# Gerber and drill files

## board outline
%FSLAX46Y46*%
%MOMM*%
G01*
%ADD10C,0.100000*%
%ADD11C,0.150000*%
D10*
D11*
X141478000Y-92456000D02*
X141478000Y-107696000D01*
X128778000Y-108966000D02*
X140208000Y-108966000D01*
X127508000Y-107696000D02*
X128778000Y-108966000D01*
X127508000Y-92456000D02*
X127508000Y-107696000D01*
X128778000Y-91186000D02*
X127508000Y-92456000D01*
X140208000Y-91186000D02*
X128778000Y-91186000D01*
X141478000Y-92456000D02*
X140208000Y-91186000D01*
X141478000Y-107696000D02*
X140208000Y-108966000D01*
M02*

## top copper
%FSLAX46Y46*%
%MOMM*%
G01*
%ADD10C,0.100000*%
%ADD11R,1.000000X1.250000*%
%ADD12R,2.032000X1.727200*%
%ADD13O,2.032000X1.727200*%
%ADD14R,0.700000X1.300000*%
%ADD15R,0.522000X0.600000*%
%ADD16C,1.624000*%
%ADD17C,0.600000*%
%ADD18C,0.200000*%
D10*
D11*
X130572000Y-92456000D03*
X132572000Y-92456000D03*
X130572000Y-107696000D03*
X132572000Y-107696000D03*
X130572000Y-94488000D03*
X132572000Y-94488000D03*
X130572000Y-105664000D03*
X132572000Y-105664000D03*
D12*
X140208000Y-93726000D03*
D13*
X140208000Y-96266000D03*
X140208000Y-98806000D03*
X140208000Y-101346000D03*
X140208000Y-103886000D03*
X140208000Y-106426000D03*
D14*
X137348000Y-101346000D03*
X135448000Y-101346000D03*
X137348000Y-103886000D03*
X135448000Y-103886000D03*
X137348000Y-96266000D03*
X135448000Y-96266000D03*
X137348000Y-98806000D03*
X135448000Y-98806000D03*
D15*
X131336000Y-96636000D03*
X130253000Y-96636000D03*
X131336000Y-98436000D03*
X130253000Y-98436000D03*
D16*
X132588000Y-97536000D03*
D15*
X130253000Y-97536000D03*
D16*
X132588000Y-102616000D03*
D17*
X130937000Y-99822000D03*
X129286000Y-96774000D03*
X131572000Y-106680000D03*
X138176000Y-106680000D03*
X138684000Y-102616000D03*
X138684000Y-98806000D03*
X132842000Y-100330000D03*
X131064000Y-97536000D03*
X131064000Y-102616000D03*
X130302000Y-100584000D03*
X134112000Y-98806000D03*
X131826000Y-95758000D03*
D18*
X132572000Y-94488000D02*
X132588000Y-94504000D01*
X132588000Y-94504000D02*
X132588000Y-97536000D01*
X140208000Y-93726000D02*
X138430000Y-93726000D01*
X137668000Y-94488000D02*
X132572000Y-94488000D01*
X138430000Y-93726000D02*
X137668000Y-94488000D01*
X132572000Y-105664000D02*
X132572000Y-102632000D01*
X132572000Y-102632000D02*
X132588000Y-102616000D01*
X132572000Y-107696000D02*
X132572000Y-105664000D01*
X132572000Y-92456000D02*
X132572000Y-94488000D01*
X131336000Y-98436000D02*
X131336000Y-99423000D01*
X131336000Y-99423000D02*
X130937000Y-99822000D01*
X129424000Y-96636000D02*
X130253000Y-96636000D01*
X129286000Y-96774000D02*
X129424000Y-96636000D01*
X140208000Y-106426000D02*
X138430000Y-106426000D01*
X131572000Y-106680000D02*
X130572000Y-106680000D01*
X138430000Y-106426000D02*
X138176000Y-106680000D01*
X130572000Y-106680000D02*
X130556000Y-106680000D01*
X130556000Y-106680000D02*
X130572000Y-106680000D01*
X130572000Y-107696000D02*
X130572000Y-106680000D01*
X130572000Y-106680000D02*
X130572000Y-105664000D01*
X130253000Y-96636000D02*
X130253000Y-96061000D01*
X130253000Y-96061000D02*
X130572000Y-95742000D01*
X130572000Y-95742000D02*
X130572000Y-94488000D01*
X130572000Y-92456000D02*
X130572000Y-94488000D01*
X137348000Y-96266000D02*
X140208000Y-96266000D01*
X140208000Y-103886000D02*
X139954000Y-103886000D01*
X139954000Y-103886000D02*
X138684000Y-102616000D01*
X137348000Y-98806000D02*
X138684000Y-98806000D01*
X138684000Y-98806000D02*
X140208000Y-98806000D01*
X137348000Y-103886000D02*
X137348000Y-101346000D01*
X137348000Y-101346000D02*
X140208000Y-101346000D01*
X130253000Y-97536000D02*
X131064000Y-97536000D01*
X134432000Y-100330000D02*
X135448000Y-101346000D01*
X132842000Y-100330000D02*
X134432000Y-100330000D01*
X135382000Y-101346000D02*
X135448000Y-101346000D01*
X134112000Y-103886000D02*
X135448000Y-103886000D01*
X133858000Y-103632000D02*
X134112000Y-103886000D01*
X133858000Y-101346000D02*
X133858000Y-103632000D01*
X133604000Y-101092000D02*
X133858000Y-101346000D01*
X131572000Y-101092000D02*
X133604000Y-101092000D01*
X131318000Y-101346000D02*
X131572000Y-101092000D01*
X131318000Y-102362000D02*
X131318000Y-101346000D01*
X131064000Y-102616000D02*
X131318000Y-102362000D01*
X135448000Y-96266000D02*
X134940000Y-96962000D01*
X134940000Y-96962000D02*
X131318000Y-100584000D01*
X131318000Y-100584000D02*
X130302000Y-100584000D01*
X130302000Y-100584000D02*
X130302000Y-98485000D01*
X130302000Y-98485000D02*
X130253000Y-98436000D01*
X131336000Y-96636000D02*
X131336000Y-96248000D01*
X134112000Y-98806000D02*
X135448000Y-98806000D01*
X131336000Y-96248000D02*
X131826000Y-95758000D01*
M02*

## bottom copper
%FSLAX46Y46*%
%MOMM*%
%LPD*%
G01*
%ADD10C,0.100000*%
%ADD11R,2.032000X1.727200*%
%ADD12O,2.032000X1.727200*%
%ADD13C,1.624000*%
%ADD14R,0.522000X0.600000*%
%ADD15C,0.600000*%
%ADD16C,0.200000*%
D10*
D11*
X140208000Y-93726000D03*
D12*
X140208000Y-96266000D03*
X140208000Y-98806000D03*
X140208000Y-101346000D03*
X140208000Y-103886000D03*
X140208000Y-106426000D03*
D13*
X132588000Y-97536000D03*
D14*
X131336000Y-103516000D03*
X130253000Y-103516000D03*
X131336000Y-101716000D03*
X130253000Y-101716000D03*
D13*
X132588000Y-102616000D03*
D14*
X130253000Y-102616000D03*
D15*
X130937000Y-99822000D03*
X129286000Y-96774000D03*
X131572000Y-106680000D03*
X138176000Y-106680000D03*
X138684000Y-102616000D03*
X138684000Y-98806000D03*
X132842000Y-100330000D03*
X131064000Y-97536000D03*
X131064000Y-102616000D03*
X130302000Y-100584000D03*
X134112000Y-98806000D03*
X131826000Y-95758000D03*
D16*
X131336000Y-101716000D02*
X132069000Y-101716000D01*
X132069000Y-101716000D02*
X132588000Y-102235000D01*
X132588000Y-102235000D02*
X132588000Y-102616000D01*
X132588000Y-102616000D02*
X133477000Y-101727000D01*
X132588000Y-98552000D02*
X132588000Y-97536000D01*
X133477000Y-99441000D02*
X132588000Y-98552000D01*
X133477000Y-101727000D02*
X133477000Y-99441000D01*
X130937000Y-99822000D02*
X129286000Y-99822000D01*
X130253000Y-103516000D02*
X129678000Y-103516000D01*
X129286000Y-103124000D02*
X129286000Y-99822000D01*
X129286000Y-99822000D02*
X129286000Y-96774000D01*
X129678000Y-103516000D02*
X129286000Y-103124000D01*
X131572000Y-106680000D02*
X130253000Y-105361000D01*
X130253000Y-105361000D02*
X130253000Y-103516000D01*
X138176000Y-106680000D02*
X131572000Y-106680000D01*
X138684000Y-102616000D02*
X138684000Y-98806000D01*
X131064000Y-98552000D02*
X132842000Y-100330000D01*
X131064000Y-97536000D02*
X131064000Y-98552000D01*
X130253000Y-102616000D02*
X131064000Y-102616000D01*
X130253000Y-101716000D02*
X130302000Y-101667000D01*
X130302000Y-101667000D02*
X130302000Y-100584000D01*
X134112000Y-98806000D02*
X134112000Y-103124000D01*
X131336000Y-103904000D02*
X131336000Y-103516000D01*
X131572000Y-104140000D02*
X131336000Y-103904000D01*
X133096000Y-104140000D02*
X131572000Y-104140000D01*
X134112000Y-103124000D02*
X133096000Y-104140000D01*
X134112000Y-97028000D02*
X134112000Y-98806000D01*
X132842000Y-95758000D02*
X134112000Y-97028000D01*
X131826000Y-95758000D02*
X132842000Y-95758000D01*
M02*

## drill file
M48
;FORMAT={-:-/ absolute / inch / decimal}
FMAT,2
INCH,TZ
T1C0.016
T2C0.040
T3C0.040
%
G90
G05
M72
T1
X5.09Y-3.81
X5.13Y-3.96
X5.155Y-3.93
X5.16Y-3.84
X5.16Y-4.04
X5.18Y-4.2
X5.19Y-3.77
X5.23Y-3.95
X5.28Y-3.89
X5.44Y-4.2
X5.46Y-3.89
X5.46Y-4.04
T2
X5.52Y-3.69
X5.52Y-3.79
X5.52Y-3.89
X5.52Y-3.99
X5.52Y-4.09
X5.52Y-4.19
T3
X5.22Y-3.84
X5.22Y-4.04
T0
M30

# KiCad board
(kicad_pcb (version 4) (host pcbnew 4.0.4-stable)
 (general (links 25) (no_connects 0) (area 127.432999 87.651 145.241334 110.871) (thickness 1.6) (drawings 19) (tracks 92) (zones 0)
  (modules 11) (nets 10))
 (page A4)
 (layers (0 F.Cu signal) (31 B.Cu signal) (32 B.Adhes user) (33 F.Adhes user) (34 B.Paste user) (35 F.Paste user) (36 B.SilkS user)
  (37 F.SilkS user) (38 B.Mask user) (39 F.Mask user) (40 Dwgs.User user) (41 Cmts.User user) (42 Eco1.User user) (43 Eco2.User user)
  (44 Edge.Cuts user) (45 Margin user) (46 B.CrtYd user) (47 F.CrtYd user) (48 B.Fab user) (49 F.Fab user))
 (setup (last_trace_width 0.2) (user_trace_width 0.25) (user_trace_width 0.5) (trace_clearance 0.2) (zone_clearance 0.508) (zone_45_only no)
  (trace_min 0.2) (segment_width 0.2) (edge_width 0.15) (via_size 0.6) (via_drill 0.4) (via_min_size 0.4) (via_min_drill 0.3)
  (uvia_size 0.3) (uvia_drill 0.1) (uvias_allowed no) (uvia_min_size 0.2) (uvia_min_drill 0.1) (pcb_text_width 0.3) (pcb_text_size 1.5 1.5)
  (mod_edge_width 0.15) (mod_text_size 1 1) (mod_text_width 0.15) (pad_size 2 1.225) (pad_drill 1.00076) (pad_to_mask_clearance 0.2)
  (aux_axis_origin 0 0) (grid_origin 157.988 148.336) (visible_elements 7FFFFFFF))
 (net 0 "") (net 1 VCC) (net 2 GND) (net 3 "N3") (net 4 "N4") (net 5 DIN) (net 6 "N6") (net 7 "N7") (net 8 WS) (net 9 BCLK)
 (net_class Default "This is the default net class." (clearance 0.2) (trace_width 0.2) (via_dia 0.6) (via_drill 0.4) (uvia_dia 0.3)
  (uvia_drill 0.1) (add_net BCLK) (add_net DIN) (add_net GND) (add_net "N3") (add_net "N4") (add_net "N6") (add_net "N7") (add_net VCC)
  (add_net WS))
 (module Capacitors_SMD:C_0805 (layer F.Cu) (at 131.572 92.456)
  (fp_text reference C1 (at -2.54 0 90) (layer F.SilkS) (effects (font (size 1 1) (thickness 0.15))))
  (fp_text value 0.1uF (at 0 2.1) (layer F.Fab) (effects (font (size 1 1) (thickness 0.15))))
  (pad 1 smd rect (at -1 0) (size 1 1.25) (layers F.Cu F.Paste F.Mask) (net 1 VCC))
  (pad 2 smd rect (at 1 0) (size 1 1.25) (layers F.Cu F.Paste F.Mask) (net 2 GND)))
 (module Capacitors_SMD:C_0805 (layer F.Cu) (at 131.572 107.696)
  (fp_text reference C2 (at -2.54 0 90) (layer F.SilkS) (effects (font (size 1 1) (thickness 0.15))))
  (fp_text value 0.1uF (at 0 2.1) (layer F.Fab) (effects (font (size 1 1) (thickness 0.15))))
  (pad 1 smd rect (at -1 0) (size 1 1.25) (layers F.Cu F.Paste F.Mask) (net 1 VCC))
  (pad 2 smd rect (at 1 0) (size 1 1.25) (layers F.Cu F.Paste F.Mask) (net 2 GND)))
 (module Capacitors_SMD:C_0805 (layer F.Cu) (at 131.572 94.488)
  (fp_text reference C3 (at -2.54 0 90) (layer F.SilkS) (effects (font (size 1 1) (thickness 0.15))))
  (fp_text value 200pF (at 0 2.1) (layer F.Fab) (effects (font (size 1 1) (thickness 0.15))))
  (pad 1 smd rect (at -1 0) (size 1 1.25) (layers F.Cu F.Paste F.Mask) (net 1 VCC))
  (pad 2 smd rect (at 1 0) (size 1 1.25) (layers F.Cu F.Paste F.Mask) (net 2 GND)))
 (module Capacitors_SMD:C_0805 (layer F.Cu) (at 131.572 105.664)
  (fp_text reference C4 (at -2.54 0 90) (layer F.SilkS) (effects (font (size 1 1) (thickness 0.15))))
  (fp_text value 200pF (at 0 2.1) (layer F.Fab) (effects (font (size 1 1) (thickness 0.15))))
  (pad 1 smd rect (at -1 0) (size 1 1.25) (layers F.Cu F.Paste F.Mask) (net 1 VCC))
  (pad 2 smd rect (at 1 0) (size 1 1.25) (layers F.Cu F.Paste F.Mask) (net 2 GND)))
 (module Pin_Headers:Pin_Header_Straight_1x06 (layer F.Cu) (at 140.208 93.726)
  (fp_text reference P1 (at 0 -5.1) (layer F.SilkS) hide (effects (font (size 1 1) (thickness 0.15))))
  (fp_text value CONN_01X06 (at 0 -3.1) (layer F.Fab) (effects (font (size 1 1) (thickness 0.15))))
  (pad 1 thru_hole rect (at 0 0) (size 2.032 1.7272) (drill 1.016) (layers *.Cu *.Mask F.SilkS) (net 2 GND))
  (pad 2 thru_hole oval (at 0 2.54) (size 2.032 1.7272) (drill 1.016) (layers *.Cu *.Mask F.SilkS) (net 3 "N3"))
  (pad 3 thru_hole oval (at 0 5.08) (size 2.032 1.7272) (drill 1.016) (layers *.Cu *.Mask F.SilkS) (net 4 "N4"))
  (pad 4 thru_hole oval (at 0 7.62) (size 2.032 1.7272) (drill 1.016) (layers *.Cu *.Mask F.SilkS) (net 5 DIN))
  (pad 5 thru_hole oval (at 0 10.16) (size 2.032 1.7272) (drill 1.016) (layers *.Cu *.Mask F.SilkS) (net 4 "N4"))
  (pad 6 thru_hole oval (at 0 12.7) (size 2.032 1.7272) (drill 1.016) (layers *.Cu *.Mask F.SilkS) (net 1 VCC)))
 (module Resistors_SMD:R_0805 (layer F.Cu) (at 136.398 101.346 180)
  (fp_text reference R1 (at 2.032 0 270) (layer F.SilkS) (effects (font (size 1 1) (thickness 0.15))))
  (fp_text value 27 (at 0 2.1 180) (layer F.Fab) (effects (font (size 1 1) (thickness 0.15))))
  (pad 1 smd rect (at -0.95 0 180) (size 0.7 1.3) (layers F.Cu F.Paste F.Mask) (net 5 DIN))
  (pad 2 smd rect (at 0.95 0 180) (size 0.7 1.3) (layers F.Cu F.Paste F.Mask) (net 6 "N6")))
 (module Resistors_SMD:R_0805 (layer F.Cu) (at 136.398 103.886 180)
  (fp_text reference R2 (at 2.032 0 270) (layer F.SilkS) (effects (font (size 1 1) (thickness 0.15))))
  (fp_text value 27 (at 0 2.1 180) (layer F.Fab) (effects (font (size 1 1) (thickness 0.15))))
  (pad 1 smd rect (at -0.95 0 180) (size 0.7 1.3) (layers F.Cu F.Paste F.Mask) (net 5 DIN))
  (pad 2 smd rect (at 0.95 0 180) (size 0.7 1.3) (layers F.Cu F.Paste F.Mask) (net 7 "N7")))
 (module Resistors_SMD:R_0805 (layer F.Cu) (at 136.398 96.266 180)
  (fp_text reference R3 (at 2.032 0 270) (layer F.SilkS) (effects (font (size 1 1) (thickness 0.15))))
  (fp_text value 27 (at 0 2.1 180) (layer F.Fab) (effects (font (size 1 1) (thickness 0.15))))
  (pad 1 smd rect (at -0.95 0 180) (size 0.7 1.3) (layers F.Cu F.Paste F.Mask) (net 3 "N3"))
  (pad 2 smd rect (at 0.95 0 180) (size 0.7 1.3) (layers F.Cu F.Paste F.Mask) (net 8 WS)))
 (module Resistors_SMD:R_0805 (layer F.Cu) (at 136.398 98.806 180)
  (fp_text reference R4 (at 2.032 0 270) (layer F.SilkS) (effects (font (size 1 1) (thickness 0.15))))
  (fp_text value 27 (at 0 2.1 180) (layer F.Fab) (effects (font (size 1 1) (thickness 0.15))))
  (pad 1 smd rect (at -0.95 0 180) (size 0.7 1.3) (layers F.Cu F.Paste F.Mask) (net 4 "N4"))
  (pad 2 smd rect (at 0.95 0 180) (size 0.7 1.3) (layers F.Cu F.Paste F.Mask) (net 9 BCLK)))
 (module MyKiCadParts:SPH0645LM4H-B (layer F.Cu) (at 132.588 97.536 90)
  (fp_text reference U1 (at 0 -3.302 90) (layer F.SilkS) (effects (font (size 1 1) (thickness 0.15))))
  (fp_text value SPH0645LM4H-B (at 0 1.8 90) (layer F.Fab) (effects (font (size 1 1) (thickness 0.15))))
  (pad 4 smd rect (at 0.9 -1.252 90) (size 0.6 0.522) (layers F.Cu F.Paste F.Mask) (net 9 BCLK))
  (pad 5 smd rect (at 0.9 -2.335 90) (size 0.6 0.522) (layers F.Cu F.Paste F.Mask) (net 1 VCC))
  (pad 2 smd rect (at -0.9 -1.252 90) (size 0.6 0.522) (layers F.Cu F.Paste F.Mask) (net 1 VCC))
  (pad 1 smd rect (at -0.9 -2.335 90) (size 0.6 0.522) (layers F.Cu F.Paste F.Mask) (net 8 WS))
  (pad 3 thru_hole circle (at 0 0 90) (size 1.624 1.624) (drill 1.024) (layers *.Cu *.Mask F.SilkS) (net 2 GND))
  (pad 6 smd rect (at 0 -2.335 90) (size 0.6 0.522) (layers F.Cu F.Paste F.Mask) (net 6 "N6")))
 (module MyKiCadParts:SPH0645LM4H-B (layer B.Cu) (at 132.588 102.616 270)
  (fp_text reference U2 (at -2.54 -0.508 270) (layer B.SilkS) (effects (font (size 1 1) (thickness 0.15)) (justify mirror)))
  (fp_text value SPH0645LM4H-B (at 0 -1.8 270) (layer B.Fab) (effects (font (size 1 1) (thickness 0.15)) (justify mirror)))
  (pad 4 smd rect (at 0.9 1.252 270) (size 0.6 0.522) (layers B.Cu B.Paste B.Mask) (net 9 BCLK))
  (pad 5 smd rect (at 0.9 2.335 270) (size 0.6 0.522) (layers B.Cu B.Paste B.Mask) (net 1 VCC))
  (pad 2 smd rect (at -0.9 1.252 270) (size 0.6 0.522) (layers B.Cu B.Paste B.Mask) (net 2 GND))
  (pad 1 smd rect (at -0.9 2.335 270) (size 0.6 0.522) (layers B.Cu B.Paste B.Mask) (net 8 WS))
  (pad 3 thru_hole circle (at 0 0 270) (size 1.624 1.624) (drill 1.024) (layers *.Cu *.Mask B.SilkS) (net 2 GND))
  (pad 6 smd rect (at 0 2.335 270) (size 0.6 0.522) (layers B.Cu B.Paste B.Mask) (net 7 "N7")))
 (gr_line (start 141.478 92.456) (end 141.478 107.696) (angle 90) (layer Edge.Cuts) (width 0.15))
 (gr_line (start 128.778 108.966) (end 140.208 108.966) (angle 90) (layer Edge.Cuts) (width 0.15))
 (gr_line (start 127.508 107.696) (end 128.778 108.966) (angle 90) (layer Edge.Cuts) (width 0.15))
 (gr_line (start 127.508 92.456) (end 127.508 107.696) (angle 90) (layer Edge.Cuts) (width 0.15))
 (gr_line (start 128.778 91.186) (end 127.508 92.456) (angle 90) (layer Edge.Cuts) (width 0.15))
 (gr_line (start 140.208 91.186) (end 128.778 91.186) (angle 90) (layer Edge.Cuts) (width 0.15))
 (gr_line (start 141.478 92.456) (end 140.208 91.186) (angle 90) (layer Edge.Cuts) (width 0.15))
 (gr_line (start 141.478 107.696) (end 140.208 108.966) (angle 90) (layer Edge.Cuts) (width 0.15))
 (segment (start 131.336 101.716) (end 132.069 101.716) (width 0.2) (layer B.Cu) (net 2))
 (segment (start 132.069 101.716) (end 132.588 102.235) (width 0.2) (layer B.Cu) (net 2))
 (segment (start 132.588 102.235) (end 132.588 102.616) (width 0.2) (layer B.Cu) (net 2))
 (segment (start 132.588 102.616) (end 133.477 101.727) (width 0.2) (layer B.Cu) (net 2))
 (segment (start 132.588 98.552) (end 132.588 97.536) (width 0.2) (layer B.Cu) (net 2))
 (segment (start 133.477 99.441) (end 132.588 98.552) (width 0.2) (layer B.Cu) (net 2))
 (segment (start 133.477 101.727) (end 133.477 99.441) (width 0.2) (layer B.Cu) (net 2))
 (segment (start 132.572 94.488) (end 132.588 94.504) (width 0.2) (layer F.Cu) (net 2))
 (segment (start 132.588 94.504) (end 132.588 97.536) (width 0.2) (layer F.Cu) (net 2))
 (segment (start 140.208 93.726) (end 138.43 93.726) (width 0.2) (layer F.Cu) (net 2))
 (segment (start 137.668 94.488) (end 132.572 94.488) (width 0.2) (layer F.Cu) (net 2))
 (segment (start 138.43 93.726) (end 137.668 94.488) (width 0.2) (layer F.Cu) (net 2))
 (segment (start 132.572 105.664) (end 132.572 102.632) (width 0.2) (layer F.Cu) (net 2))
 (segment (start 132.572 102.632) (end 132.588 102.616) (width 0.2) (layer F.Cu) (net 2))
 (segment (start 132.572 107.696) (end 132.572 105.664) (width 0.2) (layer F.Cu) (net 2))
 (segment (start 132.572 92.456) (end 132.572 94.488) (width 0.2) (layer F.Cu) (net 2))
 (segment (start 131.336 98.436) (end 131.336 99.423) (width 0.2) (layer F.Cu) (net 1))
 (segment (start 130.937 99.822) (end 129.286 99.822) (width 0.2) (layer B.Cu) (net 1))
 (via (at 130.937 99.822) (size 0.6) (drill 0.4) (layers F.Cu B.Cu) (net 1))
 (segment (start 131.336 99.423) (end 130.937 99.822) (width 0.2) (layer F.Cu) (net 1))
 (segment (start 130.253 103.516) (end 129.678 103.516) (width 0.2) (layer B.Cu) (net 1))
 (segment (start 129.424 96.636) (end 130.253 96.636) (width 0.2) (layer F.Cu) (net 1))
 (segment (start 129.286 96.774) (end 129.424 96.636) (width 0.2) (layer F.Cu) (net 1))
 (via (at 129.286 96.774) (size 0.6) (drill 0.4) (layers F.Cu B.Cu) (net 1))
 (segment (start 129.286 103.124) (end 129.286 99.822) (width 0.2) (layer B.Cu) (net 1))
 (segment (start 129.286 99.822) (end 129.286 96.774) (width 0.2) (layer B.Cu) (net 1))
 (segment (start 129.678 103.516) (end 129.286 103.124) (width 0.2) (layer B.Cu) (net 1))
 (segment (start 131.572 106.68) (end 130.253 105.361) (width 0.2) (layer B.Cu) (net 1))
 (segment (start 130.253 105.361) (end 130.253 103.516) (width 0.2) (layer B.Cu) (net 1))
 (segment (start 140.208 106.426) (end 138.43 106.426) (width 0.2) (layer F.Cu) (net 1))
 (segment (start 131.572 106.68) (end 130.572 106.68) (width 0.2) (layer F.Cu) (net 1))
 (via (at 131.572 106.68) (size 0.6) (drill 0.4) (layers F.Cu B.Cu) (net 1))
 (segment (start 138.176 106.68) (end 131.572 106.68) (width 0.2) (layer B.Cu) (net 1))
 (via (at 138.176 106.68) (size 0.6) (drill 0.4) (layers F.Cu B.Cu) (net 1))
 (segment (start 138.43 106.426) (end 138.176 106.68) (width 0.2) (layer F.Cu) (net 1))
 (segment (start 130.572 106.68) (end 130.556 106.68) (width 0.2) (layer F.Cu) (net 1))
 (segment (start 130.556 106.68) (end 130.572 106.68) (width 0.2) (layer F.Cu) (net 1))
 (segment (start 130.572 107.696) (end 130.572 106.68) (width 0.2) (layer F.Cu) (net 1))
 (segment (start 130.572 106.68) (end 130.572 105.664) (width 0.2) (layer F.Cu) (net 1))
 (segment (start 130.253 96.636) (end 130.253 96.061) (width 0.2) (layer F.Cu) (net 1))
 (segment (start 130.253 96.061) (end 130.572 95.742) (width 0.2) (layer F.Cu) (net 1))
 (segment (start 130.572 95.742) (end 130.572 94.488) (width 0.2) (layer F.Cu) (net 1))
 (segment (start 130.572 92.456) (end 130.572 94.488) (width 0.2) (layer F.Cu) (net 1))
 (segment (start 137.348 96.266) (end 140.208 96.266) (width 0.2) (layer F.Cu) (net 3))
 (segment (start 140.208 103.886) (end 139.954 103.886) (width 0.2) (layer F.Cu) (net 4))
 (segment (start 139.954 103.886) (end 138.684 102.616) (width 0.2) (layer F.Cu) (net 4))
 (via (at 138.684 102.616) (size 0.6) (drill 0.4) (layers F.Cu B.Cu) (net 4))
 (segment (start 138.684 102.616) (end 138.684 98.806) (width 0.2) (layer B.Cu) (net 4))
 (via (at 138.684 98.806) (size 0.6) (drill 0.4) (layers F.Cu B.Cu) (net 4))
 (segment (start 137.348 98.806) (end 138.684 98.806) (width 0.2) (layer F.Cu) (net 4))
 (segment (start 138.684 98.806) (end 140.208 98.806) (width 0.2) (layer F.Cu) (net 4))
 (segment (start 137.348 103.886) (end 137.348 101.346) (width 0.2) (layer F.Cu) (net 5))
 (segment (start 137.348 101.346) (end 140.208 101.346) (width 0.2) (layer F.Cu) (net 5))
 (segment (start 130.253 97.536) (end 131.064 97.536) (width 0.2) (layer F.Cu) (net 6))
 (segment (start 134.432 100.33) (end 135.448 101.346) (width 0.2) (layer F.Cu) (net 6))
 (segment (start 132.842 100.33) (end 134.432 100.33) (width 0.2) (layer F.Cu) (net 6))
 (via (at 132.842 100.33) (size 0.6) (drill 0.4) (layers F.Cu B.Cu) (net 6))
 (segment (start 131.064 98.552) (end 132.842 100.33) (width 0.2) (layer B.Cu) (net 6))
 (segment (start 131.064 97.536) (end 131.064 98.552) (width 0.2) (layer B.Cu) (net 6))
 (via (at 131.064 97.536) (size 0.6) (drill 0.4) (layers F.Cu B.Cu) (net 6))
 (segment (start 135.382 101.346) (end 135.448 101.346) (width 0.2) (layer F.Cu) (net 6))
 (segment (start 130.253 102.616) (end 131.064 102.616) (width 0.2) (layer B.Cu) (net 7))
 (segment (start 134.112 103.886) (end 135.448 103.886) (width 0.2) (layer F.Cu) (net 7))
 (segment (start 133.858 103.632) (end 134.112 103.886) (width 0.2) (layer F.Cu) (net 7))
 (segment (start 133.858 101.346) (end 133.858 103.632) (width 0.2) (layer F.Cu) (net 7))
 (segment (start 133.604 101.092) (end 133.858 101.346) (width 0.2) (layer F.Cu) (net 7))
 (segment (start 131.572 101.092) (end 133.604 101.092) (width 0.2) (layer F.Cu) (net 7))
 (segment (start 131.318 101.346) (end 131.572 101.092) (width 0.2) (layer F.Cu) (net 7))
 (segment (start 131.318 102.362) (end 131.318 101.346) (width 0.2) (layer F.Cu) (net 7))
 (segment (start 131.064 102.616) (end 131.318 102.362) (width 0.2) (layer F.Cu) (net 7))
 (via (at 131.064 102.616) (size 0.6) (drill 0.4) (layers F.Cu B.Cu) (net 7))
 (segment (start 135.448 96.266) (end 134.94 96.962) (width 0.2) (layer F.Cu) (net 8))
 (segment (start 134.94 96.962) (end 131.318 100.584) (width 0.2) (layer F.Cu) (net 8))
 (segment (start 131.318 100.584) (end 130.302 100.584) (width 0.2) (layer F.Cu) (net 8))
 (segment (start 130.253 101.716) (end 130.302 101.667) (width 0.2) (layer B.Cu) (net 8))
 (segment (start 130.302 101.667) (end 130.302 100.584) (width 0.2) (layer B.Cu) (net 8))
 (via (at 130.302 100.584) (size 0.6) (drill 0.4) (layers F.Cu B.Cu) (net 8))
 (segment (start 130.302 100.584) (end 130.302 98.485) (width 0.2) (layer F.Cu) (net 8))
 (segment (start 130.302 98.485) (end 130.253 98.436) (width 0.2) (layer F.Cu) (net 8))
 (segment (start 134.112 98.806) (end 134.112 103.124) (width 0.2) (layer B.Cu) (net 9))
 (segment (start 131.336 103.904) (end 131.336 103.516) (width 0.2) (layer B.Cu) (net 9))
 (segment (start 131.572 104.14) (end 131.336 103.904) (width 0.2) (layer B.Cu) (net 9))
 (segment (start 133.096 104.14) (end 131.572 104.14) (width 0.2) (layer B.Cu) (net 9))
 (segment (start 134.112 103.124) (end 133.096 104.14) (width 0.2) (layer B.Cu) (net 9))
 (segment (start 131.336 96.636) (end 131.336 96.248) (width 0.2) (layer F.Cu) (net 9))
 (segment (start 134.112 98.806) (end 135.448 98.806) (width 0.2) (layer F.Cu) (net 9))
 (via (at 134.112 98.806) (size 0.6) (drill 0.4) (layers F.Cu B.Cu) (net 9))
 (segment (start 134.112 97.028) (end 134.112 98.806) (width 0.2) (layer B.Cu) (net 9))
 (segment (start 132.842 95.758) (end 134.112 97.028) (width 0.2) (layer B.Cu) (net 9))
 (segment (start 131.826 95.758) (end 132.842 95.758) (width 0.2) (layer B.Cu) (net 9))
 (via (at 131.826 95.758) (size 0.6) (drill 0.4) (layers F.Cu B.Cu) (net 9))
 (segment (start 131.336 96.248) (end 131.826 95.758) (width 0.2) (layer F.Cu) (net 9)))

